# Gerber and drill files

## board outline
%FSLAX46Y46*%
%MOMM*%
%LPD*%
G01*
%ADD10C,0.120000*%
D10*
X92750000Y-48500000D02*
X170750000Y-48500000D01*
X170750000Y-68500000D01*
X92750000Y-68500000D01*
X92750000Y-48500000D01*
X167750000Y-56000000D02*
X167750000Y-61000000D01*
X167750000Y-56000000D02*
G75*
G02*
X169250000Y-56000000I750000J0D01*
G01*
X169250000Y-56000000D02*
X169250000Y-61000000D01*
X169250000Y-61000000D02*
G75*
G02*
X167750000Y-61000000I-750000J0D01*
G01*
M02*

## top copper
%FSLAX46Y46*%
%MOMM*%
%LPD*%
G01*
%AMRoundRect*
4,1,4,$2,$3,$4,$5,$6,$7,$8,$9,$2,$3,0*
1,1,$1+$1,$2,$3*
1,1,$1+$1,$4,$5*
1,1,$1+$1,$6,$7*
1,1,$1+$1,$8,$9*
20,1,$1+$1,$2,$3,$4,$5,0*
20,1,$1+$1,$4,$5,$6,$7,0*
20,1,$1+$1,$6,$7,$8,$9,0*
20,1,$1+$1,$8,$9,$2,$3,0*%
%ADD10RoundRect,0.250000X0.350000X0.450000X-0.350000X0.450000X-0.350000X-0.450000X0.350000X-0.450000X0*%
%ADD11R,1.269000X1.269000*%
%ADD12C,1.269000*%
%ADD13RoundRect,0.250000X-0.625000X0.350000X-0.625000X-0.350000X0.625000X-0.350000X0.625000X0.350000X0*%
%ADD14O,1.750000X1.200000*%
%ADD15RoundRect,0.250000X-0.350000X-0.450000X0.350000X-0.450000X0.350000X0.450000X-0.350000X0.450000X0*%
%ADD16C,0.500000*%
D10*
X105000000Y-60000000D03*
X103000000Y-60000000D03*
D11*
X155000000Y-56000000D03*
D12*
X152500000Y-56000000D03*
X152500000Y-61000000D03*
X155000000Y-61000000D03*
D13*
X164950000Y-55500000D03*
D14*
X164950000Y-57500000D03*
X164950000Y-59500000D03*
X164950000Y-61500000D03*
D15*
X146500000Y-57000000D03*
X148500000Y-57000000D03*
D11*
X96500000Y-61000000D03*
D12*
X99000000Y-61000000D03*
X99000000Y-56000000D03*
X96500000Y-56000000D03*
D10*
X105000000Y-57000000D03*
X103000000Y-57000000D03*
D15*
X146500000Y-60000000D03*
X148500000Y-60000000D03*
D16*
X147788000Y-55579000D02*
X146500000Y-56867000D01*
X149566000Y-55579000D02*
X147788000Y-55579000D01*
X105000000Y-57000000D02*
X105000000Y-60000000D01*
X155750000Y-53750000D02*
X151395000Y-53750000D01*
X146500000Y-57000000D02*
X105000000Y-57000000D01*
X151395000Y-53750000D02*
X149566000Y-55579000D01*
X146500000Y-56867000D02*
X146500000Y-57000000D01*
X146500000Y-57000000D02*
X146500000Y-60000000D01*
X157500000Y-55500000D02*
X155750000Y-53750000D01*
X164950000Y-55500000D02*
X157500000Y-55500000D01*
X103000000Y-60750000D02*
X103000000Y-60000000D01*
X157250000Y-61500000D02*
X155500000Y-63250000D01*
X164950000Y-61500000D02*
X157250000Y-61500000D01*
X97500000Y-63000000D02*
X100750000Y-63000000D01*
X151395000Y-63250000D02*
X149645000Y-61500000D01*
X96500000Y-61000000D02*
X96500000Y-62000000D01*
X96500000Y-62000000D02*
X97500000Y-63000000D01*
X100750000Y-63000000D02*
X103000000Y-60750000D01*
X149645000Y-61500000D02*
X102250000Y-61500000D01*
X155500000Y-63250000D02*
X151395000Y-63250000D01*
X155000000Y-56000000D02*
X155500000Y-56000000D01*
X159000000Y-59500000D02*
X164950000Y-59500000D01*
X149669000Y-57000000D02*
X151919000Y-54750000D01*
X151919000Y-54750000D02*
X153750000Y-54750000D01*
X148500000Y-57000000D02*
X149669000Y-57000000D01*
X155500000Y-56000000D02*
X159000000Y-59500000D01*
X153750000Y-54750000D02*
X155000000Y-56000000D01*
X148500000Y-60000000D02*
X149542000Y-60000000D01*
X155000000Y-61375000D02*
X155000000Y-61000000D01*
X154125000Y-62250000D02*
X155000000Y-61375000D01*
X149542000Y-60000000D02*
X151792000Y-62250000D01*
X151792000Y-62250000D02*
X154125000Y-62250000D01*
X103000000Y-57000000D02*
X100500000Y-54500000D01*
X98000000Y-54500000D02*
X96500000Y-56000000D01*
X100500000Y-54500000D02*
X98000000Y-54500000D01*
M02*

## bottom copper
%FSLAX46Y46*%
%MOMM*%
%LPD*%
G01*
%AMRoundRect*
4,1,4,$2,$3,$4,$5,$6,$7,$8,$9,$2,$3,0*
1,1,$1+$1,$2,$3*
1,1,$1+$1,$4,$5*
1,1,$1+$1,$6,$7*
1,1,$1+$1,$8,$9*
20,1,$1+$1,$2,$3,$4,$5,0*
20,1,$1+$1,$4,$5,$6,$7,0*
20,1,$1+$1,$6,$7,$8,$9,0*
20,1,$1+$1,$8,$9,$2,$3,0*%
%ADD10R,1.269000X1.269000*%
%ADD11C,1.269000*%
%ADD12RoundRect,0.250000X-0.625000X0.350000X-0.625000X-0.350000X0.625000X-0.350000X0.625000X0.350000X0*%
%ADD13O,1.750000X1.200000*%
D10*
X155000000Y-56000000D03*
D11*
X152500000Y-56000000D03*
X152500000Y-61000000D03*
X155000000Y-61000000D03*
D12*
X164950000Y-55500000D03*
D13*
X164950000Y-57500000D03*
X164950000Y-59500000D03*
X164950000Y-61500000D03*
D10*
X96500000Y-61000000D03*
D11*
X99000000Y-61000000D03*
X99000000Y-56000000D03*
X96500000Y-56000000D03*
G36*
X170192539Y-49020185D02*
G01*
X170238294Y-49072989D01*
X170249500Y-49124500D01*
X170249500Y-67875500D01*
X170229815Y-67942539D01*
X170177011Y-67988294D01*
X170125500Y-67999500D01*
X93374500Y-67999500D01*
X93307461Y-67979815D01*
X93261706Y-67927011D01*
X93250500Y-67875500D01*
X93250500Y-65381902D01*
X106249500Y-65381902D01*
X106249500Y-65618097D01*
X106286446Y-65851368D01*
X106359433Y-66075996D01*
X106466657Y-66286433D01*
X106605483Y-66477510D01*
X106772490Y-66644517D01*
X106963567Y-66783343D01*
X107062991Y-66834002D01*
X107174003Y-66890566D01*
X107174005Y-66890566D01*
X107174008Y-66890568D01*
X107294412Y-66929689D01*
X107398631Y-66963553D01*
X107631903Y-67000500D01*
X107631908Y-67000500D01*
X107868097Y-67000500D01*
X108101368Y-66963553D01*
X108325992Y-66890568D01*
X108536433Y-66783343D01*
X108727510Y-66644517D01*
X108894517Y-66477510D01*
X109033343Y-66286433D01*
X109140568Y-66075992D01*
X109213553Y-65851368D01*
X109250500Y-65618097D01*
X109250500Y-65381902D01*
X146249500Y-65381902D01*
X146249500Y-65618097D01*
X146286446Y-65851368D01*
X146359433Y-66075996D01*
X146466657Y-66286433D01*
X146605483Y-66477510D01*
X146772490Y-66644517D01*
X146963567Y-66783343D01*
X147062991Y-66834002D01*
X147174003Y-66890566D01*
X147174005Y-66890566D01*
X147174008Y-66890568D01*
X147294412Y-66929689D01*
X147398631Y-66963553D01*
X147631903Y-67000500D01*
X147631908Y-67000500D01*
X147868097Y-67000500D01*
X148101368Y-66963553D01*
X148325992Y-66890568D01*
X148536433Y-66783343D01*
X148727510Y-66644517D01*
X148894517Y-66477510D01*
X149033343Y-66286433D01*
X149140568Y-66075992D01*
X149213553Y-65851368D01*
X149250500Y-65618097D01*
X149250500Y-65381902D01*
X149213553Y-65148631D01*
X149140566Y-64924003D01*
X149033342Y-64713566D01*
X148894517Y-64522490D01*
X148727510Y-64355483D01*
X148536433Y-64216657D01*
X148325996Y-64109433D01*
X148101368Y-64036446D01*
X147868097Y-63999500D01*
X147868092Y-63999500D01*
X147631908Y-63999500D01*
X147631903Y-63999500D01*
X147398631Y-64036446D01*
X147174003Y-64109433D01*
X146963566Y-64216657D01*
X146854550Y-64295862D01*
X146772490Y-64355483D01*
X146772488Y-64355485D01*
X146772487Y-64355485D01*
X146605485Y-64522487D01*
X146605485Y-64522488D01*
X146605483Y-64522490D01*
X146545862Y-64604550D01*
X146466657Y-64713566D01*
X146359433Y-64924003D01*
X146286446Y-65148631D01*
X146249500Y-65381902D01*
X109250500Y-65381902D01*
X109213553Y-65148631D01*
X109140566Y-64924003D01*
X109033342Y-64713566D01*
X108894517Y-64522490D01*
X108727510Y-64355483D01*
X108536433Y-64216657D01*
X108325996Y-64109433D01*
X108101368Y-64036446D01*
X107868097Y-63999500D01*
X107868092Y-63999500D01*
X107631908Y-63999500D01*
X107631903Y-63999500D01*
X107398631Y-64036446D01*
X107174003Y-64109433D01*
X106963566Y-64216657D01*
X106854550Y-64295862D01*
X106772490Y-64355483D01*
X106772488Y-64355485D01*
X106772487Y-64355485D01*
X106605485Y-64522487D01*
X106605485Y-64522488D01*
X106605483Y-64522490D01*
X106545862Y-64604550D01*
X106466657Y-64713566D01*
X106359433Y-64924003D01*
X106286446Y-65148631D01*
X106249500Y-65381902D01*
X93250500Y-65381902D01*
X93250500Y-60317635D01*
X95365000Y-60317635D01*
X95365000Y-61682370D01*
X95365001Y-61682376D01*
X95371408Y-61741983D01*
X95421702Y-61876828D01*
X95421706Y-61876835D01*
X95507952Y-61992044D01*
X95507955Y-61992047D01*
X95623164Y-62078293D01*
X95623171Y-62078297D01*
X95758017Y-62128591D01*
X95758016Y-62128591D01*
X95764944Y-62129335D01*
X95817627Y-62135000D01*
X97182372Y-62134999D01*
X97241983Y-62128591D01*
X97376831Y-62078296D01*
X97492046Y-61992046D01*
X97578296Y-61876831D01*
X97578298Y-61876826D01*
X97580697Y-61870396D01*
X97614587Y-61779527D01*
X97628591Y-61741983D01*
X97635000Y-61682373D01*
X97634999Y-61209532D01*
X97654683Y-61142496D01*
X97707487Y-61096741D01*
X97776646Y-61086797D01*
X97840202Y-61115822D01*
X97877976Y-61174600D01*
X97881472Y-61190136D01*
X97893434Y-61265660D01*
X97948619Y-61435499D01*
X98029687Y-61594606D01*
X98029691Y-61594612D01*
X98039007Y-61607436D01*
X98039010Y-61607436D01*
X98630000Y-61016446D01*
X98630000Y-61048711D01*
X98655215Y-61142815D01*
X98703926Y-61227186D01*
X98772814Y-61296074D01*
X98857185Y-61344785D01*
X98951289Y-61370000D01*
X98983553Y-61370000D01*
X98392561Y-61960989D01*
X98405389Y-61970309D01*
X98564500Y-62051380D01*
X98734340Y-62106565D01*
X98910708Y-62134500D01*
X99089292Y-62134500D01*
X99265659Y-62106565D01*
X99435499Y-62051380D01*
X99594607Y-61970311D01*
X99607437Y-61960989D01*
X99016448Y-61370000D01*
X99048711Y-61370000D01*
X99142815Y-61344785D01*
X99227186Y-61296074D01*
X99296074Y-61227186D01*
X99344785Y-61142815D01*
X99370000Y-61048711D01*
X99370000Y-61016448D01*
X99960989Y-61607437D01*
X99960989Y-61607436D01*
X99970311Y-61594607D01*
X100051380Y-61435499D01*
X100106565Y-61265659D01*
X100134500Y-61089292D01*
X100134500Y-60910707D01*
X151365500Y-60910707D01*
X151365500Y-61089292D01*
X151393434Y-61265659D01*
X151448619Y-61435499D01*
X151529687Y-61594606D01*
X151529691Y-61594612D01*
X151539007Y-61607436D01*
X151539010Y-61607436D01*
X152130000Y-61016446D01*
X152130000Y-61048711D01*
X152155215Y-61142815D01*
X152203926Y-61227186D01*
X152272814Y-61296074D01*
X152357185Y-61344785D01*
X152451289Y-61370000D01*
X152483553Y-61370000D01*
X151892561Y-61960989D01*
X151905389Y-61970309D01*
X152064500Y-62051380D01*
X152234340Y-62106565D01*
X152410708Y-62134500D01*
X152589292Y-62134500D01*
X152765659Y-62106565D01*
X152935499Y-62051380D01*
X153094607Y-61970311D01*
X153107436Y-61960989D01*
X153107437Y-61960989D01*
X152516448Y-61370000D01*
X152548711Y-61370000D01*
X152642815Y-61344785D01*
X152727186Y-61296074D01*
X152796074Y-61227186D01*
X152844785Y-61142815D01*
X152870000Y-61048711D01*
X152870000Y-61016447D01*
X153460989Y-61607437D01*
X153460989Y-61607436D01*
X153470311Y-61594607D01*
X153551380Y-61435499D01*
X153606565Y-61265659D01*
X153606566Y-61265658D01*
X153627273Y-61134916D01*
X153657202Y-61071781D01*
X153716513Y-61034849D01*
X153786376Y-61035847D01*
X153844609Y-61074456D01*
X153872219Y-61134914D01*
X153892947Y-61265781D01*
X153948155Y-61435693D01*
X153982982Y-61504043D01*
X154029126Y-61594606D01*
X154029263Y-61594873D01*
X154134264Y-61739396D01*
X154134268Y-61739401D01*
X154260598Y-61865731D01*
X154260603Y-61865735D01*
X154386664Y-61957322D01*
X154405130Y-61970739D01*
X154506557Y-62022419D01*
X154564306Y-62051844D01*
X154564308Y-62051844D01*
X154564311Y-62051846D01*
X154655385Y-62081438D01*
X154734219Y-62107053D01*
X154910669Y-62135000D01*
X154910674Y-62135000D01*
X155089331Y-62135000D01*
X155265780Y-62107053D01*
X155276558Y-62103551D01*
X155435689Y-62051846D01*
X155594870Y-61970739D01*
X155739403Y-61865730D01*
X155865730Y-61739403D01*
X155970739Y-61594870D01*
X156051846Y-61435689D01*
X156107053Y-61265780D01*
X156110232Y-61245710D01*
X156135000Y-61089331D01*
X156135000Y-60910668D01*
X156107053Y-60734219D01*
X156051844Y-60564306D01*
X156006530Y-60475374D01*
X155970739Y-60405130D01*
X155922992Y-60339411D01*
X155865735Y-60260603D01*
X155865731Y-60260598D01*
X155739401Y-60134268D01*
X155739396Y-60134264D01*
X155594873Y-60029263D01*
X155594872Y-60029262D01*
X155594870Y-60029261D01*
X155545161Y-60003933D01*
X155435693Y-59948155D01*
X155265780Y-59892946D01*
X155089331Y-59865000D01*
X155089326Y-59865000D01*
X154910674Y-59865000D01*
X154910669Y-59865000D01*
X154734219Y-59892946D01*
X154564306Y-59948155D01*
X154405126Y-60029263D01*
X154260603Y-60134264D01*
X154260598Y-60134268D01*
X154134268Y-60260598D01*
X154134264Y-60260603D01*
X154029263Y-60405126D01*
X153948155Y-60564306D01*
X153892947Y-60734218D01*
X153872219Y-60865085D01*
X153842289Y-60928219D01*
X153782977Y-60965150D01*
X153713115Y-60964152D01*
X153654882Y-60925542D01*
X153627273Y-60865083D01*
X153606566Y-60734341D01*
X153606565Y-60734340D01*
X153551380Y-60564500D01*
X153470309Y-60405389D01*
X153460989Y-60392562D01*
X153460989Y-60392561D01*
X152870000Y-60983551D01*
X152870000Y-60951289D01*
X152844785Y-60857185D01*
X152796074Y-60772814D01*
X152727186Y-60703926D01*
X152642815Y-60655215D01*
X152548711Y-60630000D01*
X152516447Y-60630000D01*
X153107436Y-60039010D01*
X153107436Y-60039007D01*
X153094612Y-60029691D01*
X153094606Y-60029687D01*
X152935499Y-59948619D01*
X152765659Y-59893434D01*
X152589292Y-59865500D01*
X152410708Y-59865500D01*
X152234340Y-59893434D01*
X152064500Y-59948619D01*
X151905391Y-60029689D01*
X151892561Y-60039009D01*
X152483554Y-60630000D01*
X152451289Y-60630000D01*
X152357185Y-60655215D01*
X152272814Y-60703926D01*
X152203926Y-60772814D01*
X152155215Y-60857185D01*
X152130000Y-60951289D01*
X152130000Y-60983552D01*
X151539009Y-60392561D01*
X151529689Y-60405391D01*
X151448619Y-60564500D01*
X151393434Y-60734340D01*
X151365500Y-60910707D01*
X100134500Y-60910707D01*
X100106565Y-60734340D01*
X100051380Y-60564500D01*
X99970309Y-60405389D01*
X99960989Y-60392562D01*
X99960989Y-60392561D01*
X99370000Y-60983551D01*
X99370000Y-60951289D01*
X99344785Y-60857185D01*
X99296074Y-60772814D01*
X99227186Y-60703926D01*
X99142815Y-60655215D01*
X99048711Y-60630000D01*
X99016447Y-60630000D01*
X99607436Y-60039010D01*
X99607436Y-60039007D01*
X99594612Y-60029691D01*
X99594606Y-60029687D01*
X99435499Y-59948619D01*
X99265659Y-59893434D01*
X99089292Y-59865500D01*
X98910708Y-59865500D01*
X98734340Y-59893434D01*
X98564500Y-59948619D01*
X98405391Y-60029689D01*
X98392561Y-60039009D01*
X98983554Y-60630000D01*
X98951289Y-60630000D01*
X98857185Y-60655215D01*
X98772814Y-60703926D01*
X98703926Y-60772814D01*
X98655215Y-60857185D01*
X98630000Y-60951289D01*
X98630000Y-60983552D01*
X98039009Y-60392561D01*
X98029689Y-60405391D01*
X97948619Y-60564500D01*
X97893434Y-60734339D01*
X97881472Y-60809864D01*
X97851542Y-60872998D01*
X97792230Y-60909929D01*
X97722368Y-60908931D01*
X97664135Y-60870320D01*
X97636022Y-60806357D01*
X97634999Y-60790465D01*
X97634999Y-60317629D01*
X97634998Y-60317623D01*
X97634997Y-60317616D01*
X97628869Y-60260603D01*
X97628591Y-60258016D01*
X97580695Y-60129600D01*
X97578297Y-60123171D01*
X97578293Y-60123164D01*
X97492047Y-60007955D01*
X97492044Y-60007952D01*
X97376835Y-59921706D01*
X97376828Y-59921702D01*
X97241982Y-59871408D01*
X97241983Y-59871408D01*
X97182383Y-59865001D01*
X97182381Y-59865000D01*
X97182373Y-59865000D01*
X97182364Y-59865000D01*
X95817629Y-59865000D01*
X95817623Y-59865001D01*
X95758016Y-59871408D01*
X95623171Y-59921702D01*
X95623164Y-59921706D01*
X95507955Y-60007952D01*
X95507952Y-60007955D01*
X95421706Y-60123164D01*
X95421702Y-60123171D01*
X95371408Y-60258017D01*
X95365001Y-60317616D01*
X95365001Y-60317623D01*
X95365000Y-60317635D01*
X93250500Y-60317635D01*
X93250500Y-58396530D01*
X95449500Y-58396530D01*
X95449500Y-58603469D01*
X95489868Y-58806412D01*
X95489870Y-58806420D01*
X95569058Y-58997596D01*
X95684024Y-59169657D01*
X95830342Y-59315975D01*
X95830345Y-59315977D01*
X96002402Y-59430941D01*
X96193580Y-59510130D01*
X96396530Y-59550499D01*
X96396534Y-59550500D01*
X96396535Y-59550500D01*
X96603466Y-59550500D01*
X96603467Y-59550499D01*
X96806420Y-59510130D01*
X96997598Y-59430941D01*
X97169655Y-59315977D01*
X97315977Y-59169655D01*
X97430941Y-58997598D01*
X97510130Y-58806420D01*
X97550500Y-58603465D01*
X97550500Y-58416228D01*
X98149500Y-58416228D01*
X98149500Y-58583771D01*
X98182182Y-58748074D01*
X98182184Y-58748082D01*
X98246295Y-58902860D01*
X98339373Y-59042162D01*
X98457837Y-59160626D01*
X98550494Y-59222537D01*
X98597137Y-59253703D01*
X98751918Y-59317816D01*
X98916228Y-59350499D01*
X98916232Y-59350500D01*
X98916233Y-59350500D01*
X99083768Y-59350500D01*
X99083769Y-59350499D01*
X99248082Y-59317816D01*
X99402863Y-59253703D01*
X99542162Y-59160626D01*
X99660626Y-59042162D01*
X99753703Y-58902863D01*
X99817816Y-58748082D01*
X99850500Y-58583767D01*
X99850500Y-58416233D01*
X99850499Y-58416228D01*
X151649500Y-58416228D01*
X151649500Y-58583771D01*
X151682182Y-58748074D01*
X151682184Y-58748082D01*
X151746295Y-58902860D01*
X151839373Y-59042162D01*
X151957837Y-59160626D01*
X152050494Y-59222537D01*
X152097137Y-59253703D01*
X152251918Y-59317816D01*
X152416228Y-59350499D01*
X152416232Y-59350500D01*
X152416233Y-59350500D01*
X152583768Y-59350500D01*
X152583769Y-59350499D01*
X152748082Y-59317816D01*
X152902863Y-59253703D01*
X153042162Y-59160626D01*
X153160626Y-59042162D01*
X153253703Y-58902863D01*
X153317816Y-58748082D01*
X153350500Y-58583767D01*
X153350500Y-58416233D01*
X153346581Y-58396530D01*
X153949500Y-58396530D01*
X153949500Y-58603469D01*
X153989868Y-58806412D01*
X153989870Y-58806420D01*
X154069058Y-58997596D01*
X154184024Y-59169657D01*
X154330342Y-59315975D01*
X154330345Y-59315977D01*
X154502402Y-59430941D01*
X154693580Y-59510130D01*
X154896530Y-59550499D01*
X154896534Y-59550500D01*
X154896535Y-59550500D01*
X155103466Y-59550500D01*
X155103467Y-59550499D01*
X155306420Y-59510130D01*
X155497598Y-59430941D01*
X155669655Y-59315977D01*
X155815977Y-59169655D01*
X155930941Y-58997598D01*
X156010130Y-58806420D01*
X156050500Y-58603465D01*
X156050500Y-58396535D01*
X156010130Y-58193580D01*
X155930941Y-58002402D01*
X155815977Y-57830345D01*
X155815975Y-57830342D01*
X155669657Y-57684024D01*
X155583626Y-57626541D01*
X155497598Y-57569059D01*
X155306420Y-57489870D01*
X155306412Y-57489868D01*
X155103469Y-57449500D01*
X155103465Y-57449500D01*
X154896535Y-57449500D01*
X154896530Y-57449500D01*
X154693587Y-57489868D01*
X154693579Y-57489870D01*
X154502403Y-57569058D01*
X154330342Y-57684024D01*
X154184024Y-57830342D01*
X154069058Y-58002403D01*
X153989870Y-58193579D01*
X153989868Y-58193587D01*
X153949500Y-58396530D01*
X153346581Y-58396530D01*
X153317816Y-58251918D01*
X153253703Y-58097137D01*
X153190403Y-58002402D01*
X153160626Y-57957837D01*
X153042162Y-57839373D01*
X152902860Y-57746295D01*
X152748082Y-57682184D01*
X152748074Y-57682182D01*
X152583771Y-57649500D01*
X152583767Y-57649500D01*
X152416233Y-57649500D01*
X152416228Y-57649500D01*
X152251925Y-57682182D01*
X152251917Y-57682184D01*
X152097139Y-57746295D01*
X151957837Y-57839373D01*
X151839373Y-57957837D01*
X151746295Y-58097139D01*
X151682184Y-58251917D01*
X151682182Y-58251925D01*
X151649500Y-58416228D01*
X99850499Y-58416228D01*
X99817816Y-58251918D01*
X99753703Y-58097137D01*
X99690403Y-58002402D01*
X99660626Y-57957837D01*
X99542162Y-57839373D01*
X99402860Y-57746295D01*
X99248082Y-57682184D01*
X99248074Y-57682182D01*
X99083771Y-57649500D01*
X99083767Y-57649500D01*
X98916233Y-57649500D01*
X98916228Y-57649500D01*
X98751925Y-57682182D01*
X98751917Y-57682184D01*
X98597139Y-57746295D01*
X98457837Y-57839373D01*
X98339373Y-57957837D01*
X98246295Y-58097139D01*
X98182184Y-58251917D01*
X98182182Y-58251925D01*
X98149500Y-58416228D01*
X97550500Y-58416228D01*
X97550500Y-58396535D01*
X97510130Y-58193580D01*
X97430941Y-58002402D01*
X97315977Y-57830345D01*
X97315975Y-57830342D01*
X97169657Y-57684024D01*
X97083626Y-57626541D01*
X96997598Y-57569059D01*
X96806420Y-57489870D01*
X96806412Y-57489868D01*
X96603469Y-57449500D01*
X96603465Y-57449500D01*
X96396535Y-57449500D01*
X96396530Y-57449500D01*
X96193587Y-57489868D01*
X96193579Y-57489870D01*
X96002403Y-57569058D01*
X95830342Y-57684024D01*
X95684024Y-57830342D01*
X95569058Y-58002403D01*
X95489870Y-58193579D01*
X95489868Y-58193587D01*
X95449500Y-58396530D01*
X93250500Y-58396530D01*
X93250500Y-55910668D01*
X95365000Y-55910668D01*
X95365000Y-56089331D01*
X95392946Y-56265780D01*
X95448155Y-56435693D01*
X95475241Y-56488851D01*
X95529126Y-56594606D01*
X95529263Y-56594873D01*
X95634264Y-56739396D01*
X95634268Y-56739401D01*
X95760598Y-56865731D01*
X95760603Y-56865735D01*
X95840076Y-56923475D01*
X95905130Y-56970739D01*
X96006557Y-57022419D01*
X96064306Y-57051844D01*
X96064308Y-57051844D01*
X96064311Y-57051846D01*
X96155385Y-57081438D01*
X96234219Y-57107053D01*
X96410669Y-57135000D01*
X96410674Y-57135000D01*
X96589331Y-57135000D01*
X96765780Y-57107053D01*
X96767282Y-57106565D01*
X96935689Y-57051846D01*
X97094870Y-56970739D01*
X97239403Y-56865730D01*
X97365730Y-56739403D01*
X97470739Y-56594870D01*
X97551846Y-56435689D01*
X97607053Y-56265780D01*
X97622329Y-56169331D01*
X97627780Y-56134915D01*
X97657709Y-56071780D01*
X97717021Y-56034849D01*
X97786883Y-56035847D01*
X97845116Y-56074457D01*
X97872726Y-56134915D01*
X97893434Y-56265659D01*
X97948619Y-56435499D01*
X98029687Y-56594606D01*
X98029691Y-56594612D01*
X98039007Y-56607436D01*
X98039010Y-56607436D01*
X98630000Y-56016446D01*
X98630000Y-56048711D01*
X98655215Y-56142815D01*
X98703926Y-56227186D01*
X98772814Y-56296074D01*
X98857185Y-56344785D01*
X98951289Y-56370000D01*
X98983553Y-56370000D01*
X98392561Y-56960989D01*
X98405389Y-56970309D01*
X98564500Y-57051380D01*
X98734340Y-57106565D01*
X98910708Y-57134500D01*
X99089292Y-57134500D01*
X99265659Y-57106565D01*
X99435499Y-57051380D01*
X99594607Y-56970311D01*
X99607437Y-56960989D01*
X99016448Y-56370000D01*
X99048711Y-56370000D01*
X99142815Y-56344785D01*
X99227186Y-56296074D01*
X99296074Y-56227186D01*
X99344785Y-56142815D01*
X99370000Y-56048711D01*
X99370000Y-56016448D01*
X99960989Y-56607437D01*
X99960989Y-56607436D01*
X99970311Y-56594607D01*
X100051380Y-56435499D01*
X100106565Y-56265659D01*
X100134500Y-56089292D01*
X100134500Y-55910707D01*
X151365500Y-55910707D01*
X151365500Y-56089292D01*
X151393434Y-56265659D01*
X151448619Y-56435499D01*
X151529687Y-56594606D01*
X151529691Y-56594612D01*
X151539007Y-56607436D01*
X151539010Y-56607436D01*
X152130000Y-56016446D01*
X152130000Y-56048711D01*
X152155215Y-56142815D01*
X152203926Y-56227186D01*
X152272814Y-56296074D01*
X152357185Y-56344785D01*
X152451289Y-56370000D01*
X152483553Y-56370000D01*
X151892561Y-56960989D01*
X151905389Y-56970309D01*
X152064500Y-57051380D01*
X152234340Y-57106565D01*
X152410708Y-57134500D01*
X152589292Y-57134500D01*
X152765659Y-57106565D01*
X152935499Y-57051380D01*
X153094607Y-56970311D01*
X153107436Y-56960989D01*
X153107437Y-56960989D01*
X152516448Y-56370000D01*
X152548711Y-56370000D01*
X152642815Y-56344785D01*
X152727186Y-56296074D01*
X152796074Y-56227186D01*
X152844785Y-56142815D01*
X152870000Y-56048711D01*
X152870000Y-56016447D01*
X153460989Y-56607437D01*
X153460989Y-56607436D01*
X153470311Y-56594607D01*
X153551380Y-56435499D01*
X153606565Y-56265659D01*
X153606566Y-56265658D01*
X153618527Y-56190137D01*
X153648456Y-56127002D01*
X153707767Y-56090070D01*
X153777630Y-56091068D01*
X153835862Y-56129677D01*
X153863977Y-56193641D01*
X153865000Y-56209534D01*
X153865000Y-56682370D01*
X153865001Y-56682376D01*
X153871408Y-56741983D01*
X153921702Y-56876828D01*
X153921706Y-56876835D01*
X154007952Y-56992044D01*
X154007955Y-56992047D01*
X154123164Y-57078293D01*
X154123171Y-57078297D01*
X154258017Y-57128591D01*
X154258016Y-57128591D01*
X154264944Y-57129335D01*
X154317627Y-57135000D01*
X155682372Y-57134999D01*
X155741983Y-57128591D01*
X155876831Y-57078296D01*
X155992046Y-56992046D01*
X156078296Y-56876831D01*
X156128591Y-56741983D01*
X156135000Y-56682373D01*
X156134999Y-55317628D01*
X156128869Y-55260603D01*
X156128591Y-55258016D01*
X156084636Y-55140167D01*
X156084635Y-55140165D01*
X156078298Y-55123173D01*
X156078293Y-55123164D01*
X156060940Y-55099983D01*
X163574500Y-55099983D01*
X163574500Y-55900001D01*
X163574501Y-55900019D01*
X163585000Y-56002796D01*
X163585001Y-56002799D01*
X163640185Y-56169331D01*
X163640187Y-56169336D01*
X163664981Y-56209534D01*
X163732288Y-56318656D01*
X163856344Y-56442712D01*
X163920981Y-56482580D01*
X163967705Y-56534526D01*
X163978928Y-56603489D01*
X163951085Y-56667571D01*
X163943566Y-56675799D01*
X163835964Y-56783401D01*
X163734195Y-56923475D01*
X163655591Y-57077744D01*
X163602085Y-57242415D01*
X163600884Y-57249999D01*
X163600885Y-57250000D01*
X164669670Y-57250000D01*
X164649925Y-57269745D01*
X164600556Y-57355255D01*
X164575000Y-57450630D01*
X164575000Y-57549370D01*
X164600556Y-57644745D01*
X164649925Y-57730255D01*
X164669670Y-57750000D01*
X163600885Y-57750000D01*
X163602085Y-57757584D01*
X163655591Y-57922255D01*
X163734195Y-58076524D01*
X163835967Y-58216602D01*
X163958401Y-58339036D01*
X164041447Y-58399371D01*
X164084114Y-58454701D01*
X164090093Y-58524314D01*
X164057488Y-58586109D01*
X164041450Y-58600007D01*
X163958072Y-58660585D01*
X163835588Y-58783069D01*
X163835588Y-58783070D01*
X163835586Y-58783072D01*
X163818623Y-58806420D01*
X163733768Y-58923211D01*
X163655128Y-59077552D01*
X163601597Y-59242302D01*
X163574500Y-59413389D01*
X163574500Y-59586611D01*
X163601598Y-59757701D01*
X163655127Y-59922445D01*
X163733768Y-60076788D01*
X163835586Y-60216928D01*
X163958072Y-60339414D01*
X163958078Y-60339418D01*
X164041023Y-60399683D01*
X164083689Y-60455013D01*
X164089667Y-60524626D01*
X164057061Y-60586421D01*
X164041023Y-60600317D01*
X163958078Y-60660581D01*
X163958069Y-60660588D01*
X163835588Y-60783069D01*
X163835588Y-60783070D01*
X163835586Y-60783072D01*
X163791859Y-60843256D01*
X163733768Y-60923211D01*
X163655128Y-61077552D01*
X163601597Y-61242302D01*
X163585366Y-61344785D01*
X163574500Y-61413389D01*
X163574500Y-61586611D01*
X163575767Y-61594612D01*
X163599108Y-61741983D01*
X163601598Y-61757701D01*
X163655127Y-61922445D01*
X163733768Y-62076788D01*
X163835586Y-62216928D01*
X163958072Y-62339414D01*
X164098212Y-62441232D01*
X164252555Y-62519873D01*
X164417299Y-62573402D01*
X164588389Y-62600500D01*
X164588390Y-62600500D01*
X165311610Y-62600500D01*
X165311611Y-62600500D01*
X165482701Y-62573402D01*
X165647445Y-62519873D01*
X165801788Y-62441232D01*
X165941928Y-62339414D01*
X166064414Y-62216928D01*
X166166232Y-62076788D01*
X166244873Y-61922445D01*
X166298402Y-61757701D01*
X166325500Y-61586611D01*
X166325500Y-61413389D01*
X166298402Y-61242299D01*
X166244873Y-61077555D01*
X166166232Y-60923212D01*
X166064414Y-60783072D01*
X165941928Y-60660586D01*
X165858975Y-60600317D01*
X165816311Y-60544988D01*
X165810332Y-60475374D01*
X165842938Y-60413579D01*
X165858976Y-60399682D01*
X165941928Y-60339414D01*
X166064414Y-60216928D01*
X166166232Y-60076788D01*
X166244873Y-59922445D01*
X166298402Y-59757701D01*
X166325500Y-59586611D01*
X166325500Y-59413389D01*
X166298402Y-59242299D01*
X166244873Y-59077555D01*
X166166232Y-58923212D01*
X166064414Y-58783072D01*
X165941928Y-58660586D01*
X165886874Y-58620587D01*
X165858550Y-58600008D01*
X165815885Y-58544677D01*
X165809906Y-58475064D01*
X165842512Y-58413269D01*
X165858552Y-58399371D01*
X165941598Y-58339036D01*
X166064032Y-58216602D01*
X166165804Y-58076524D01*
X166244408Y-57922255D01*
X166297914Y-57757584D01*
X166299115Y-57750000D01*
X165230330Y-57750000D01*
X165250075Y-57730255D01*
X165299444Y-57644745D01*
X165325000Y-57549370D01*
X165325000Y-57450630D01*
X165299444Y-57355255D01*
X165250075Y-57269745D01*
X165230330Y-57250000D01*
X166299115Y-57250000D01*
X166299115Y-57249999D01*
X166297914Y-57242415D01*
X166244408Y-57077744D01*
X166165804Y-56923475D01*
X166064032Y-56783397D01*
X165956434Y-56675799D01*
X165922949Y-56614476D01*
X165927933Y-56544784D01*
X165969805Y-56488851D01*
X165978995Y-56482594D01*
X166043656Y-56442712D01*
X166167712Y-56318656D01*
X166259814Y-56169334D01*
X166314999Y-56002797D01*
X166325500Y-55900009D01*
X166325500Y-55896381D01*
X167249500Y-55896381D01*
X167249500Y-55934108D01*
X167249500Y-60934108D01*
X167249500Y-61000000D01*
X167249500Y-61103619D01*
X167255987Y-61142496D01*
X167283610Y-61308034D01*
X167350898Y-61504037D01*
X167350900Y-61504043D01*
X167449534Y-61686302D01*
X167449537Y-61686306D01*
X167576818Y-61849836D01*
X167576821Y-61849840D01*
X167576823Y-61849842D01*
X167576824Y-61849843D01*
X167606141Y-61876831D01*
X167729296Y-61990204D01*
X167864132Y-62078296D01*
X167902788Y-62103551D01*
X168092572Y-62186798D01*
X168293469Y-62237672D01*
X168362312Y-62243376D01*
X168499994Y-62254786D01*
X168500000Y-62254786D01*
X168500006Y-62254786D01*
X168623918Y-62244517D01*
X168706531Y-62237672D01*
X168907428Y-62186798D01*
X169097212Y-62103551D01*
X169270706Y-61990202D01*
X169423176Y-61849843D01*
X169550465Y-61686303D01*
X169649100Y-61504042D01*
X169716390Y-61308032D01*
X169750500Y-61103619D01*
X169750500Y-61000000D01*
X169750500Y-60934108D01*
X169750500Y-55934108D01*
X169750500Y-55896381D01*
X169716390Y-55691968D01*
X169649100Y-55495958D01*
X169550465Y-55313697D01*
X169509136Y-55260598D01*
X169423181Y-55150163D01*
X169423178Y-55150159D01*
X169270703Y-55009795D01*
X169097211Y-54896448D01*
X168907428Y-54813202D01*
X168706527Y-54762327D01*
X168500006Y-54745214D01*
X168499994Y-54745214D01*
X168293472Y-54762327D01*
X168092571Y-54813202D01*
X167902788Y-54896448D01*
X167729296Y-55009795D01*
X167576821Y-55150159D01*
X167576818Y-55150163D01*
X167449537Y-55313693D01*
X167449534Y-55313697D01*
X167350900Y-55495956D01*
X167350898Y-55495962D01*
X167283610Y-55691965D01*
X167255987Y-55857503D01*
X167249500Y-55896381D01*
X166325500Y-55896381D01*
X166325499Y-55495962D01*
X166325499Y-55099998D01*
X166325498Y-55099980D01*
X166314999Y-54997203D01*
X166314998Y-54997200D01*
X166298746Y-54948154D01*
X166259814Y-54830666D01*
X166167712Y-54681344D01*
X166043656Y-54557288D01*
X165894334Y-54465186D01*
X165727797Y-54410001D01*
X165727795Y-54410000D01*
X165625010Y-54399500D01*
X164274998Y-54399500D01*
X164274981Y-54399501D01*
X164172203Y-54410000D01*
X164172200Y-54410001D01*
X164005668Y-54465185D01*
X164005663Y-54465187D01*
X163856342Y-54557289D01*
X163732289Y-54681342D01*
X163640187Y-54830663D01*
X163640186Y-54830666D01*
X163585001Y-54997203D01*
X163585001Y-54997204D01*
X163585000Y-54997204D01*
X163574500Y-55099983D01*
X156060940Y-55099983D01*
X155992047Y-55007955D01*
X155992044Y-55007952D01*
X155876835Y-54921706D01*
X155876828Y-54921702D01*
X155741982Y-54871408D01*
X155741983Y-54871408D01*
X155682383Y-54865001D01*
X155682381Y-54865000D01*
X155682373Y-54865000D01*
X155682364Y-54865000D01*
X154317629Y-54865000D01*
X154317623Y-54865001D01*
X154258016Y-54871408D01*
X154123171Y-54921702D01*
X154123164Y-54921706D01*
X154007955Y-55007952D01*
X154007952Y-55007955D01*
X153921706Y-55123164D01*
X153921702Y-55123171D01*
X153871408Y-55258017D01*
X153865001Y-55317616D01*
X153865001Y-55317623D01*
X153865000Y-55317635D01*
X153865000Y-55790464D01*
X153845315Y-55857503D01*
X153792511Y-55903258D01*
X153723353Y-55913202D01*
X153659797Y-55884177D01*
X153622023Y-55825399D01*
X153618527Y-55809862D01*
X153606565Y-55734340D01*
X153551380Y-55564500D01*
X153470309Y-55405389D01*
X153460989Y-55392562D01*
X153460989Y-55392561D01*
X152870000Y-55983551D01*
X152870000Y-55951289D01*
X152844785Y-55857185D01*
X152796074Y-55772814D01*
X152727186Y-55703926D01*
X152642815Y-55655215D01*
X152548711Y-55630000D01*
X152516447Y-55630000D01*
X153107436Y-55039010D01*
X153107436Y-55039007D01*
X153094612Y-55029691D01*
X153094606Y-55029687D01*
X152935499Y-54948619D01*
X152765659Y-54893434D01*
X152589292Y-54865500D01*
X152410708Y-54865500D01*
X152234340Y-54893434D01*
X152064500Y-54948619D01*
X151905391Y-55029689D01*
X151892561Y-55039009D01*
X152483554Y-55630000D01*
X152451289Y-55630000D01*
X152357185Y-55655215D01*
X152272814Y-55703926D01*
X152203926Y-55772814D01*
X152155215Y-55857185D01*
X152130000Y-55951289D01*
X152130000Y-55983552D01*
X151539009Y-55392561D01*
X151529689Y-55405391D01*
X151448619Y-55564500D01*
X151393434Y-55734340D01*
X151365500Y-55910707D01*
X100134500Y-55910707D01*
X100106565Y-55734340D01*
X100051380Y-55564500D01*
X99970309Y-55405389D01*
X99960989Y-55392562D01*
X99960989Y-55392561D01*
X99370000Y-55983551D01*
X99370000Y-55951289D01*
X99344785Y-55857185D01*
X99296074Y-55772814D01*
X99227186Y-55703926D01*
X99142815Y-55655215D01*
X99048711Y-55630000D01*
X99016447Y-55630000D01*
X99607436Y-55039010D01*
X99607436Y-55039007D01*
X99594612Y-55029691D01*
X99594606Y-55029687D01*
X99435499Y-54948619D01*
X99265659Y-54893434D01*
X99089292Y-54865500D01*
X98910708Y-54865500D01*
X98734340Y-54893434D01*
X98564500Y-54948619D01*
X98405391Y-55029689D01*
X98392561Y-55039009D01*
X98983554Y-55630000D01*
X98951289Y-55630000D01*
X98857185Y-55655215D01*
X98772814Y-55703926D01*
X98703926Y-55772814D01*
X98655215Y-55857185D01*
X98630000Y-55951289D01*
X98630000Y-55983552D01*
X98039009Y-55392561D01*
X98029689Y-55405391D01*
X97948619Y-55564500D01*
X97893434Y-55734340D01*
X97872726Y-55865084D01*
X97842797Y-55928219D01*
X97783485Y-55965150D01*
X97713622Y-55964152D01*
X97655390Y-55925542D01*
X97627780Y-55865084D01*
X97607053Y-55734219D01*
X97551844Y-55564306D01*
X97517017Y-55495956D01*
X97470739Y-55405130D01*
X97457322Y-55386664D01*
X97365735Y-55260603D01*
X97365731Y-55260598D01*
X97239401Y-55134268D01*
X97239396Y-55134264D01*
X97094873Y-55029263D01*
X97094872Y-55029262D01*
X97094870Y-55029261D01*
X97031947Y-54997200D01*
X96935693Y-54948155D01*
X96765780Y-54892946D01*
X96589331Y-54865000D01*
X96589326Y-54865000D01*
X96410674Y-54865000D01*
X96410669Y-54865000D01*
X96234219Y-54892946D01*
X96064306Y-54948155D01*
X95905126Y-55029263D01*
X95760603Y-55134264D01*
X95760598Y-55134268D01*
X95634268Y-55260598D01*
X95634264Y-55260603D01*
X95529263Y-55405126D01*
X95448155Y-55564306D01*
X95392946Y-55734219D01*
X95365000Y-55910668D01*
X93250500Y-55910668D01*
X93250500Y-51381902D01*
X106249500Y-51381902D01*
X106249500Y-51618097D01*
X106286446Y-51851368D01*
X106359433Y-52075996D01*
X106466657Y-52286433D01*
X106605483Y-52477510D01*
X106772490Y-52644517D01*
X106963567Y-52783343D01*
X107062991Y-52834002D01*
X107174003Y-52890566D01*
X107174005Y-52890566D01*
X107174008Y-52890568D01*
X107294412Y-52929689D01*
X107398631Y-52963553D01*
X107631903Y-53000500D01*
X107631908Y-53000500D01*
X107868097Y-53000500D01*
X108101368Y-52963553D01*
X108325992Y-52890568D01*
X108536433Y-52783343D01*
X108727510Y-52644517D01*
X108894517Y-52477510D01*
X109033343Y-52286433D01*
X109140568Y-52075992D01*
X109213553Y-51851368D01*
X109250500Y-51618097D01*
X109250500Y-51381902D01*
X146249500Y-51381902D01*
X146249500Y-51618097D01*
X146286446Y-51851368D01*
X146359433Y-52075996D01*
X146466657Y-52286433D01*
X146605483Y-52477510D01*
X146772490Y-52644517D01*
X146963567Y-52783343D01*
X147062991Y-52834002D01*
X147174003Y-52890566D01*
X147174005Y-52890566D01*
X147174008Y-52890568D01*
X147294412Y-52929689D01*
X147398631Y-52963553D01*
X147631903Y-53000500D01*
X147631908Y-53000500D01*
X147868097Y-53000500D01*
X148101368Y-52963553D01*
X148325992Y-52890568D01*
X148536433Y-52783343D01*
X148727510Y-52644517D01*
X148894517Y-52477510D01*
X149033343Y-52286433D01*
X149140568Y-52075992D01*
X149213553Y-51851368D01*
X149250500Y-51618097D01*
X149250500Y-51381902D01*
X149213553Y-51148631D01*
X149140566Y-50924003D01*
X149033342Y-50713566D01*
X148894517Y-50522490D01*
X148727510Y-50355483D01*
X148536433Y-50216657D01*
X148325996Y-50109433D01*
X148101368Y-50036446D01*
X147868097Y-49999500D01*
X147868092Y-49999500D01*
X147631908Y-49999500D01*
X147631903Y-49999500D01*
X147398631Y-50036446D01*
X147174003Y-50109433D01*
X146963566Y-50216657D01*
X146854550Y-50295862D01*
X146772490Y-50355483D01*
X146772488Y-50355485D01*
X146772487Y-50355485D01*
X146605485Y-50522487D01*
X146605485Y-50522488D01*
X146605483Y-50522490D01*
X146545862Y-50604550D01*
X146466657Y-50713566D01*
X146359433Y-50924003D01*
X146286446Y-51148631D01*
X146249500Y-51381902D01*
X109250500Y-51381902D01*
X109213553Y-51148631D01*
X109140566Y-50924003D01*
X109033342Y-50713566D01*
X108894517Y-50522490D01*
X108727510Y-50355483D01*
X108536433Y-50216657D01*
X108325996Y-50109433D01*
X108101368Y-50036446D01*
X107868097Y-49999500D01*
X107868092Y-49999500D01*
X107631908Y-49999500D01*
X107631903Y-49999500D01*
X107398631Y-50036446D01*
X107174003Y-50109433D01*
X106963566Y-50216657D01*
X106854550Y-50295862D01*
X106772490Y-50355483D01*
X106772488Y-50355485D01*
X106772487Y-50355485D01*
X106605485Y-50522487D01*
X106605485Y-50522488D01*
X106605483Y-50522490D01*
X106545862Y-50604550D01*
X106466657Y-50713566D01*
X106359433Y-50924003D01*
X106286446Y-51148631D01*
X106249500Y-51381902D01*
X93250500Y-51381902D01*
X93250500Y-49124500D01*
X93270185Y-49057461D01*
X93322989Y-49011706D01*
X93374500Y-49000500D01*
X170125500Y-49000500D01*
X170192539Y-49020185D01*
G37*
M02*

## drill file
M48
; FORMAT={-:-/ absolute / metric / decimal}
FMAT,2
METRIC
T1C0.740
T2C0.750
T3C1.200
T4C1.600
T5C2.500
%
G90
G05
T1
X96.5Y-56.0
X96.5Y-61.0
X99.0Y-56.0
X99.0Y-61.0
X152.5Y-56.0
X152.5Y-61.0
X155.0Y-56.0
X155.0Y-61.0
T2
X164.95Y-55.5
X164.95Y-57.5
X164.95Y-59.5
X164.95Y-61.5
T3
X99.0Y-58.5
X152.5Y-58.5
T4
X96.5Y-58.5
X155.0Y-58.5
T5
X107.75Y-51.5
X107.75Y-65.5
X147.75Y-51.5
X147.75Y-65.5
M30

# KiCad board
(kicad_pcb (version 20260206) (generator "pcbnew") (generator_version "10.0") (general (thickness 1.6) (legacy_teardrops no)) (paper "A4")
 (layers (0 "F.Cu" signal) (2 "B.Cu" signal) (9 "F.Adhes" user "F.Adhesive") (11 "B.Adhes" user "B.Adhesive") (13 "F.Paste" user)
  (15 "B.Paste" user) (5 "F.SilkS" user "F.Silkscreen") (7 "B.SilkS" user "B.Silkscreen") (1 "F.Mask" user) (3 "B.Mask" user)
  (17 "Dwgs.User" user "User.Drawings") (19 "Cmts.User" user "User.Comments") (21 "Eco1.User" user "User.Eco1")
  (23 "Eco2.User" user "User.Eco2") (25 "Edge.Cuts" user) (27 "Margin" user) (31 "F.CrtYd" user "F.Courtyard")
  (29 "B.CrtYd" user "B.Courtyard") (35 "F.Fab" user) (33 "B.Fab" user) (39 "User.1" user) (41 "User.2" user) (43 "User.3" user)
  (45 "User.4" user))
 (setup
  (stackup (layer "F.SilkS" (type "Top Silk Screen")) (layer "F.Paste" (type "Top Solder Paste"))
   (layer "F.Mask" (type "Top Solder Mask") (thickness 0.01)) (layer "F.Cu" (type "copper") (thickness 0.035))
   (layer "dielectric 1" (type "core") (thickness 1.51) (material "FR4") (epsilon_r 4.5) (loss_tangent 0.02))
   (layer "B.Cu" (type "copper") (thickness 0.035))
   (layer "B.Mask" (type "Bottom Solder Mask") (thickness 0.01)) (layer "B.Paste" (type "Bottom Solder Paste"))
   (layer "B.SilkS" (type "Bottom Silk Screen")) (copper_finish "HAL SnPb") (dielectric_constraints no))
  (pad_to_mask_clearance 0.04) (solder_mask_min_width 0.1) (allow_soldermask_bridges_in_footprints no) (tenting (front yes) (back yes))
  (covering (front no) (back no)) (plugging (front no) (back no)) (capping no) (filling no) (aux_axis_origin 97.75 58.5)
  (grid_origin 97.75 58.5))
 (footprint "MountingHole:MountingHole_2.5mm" (layer "F.Cu") (at 107.75 51.5)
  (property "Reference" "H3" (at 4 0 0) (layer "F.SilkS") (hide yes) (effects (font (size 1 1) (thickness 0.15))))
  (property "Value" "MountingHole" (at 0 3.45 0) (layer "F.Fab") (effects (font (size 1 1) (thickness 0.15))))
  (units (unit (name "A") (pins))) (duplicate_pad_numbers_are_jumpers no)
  (pad "" np_thru_hole circle (at 0 0) (size 2.5 2.5) (drill 2.5) (layers "*.Cu" "*.Mask")))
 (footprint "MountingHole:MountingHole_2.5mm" (layer "F.Cu") (at 107.75 65.5)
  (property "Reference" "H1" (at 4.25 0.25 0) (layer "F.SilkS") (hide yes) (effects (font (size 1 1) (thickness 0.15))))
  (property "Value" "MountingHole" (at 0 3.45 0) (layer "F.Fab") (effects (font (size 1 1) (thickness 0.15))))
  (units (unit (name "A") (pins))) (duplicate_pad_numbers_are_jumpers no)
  (pad "" np_thru_hole circle (at 0 0) (size 2.5 2.5) (drill 2.5) (layers "*.Cu" "*.Mask")))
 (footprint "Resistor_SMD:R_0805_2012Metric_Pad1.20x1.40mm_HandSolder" (layer "F.Cu") (at 104 60 180)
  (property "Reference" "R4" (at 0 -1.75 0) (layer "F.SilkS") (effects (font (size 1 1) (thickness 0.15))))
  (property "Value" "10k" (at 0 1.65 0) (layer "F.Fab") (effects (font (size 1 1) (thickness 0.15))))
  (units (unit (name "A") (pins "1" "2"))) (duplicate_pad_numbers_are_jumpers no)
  (pad "1" smd roundrect (at -1 0 180) (size 1.2 1.4) (layers "F.Cu" "F.Mask" "F.Paste") (roundrect_rratio 0.208333) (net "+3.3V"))
  (pad "2" smd roundrect (at 1 0 180) (size 1.2 1.4) (layers "F.Cu" "F.Mask" "F.Paste") (roundrect_rratio 0.208333) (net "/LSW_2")))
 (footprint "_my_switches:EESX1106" (layer "F.Cu") (at 155 56 -90)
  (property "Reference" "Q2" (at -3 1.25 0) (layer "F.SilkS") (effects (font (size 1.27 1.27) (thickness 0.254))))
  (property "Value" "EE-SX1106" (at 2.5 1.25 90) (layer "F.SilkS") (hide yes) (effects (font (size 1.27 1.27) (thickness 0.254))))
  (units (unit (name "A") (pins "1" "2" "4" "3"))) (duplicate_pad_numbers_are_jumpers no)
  (pad "" np_thru_hole circle (at 2.5 0 270) (size 1.6 1.6) (drill 1.6) (layers "*.Cu" "*.Mask"))
  (pad "" np_thru_hole circle (at 2.5 2.5 270) (size 1.2 1.2) (drill 1.2) (layers "*.Cu" "*.Mask"))
  (pad "1" thru_hole rect (at 0 0 270) (size 1.269 1.269) (drill 0.74) (layers "*.Cu" "*.Mask") (remove_unused_layers no) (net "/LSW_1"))
  (pad "2" thru_hole circle (at 0 2.5 270) (size 1.269 1.269) (drill 0.74) (layers "*.Cu" "*.Mask") (remove_unused_layers no) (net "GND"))
  (pad "3" thru_hole circle (at 5 2.5 270) (size 1.269 1.269) (drill 0.74) (layers "*.Cu" "*.Mask") (remove_unused_layers no) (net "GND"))
  (pad "4" thru_hole circle (at 5 0 270) (size 1.269 1.269) (drill 0.74) (layers "*.Cu" "*.Mask") (remove_unused_layers no)
   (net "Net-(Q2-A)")))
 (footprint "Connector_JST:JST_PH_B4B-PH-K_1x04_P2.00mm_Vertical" (layer "F.Cu") (at 164.95 55.5 -90)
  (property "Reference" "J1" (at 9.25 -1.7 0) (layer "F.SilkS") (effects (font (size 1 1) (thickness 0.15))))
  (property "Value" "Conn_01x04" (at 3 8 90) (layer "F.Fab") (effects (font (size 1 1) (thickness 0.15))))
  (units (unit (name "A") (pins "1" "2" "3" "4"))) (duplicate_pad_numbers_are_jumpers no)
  (pad "1" thru_hole roundrect (at 0 0 270) (size 1.2 1.75) (drill 0.75) (layers "*.Cu" "*.Mask") (remove_unused_layers no)
   (roundrect_rratio 0.208333) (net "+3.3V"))
  (pad "2" thru_hole oval (at 2 0 270) (size 1.2 1.75) (drill 0.75) (layers "*.Cu" "*.Mask") (remove_unused_layers no) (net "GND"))
  (pad "3" thru_hole oval (at 4 0 270) (size 1.2 1.75) (drill 0.75) (layers "*.Cu" "*.Mask") (remove_unused_layers no) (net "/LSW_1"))
  (pad "4" thru_hole oval (at 6 0 270) (size 1.2 1.75) (drill 0.75) (layers "*.Cu" "*.Mask") (remove_unused_layers no) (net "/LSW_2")))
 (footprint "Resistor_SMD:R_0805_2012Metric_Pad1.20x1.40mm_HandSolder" (layer "F.Cu") (at 147.5 57)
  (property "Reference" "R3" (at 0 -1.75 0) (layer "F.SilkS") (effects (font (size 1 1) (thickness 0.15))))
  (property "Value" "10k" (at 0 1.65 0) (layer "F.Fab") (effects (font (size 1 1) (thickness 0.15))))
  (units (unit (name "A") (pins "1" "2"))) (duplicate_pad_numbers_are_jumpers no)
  (pad "1" smd roundrect (at -1 0) (size 1.2 1.4) (layers "F.Cu" "F.Mask" "F.Paste") (roundrect_rratio 0.208333) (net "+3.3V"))
  (pad "2" smd roundrect (at 1 0) (size 1.2 1.4) (layers "F.Cu" "F.Mask" "F.Paste") (roundrect_rratio 0.208333) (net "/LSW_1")))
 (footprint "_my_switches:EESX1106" (layer "F.Cu") (at 96.5 61 90)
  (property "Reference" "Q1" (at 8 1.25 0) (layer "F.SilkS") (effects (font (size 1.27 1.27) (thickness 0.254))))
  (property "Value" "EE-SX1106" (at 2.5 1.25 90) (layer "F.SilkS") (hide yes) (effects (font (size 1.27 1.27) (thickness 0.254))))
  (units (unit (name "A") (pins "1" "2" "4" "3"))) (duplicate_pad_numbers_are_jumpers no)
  (pad "" np_thru_hole circle (at 2.5 0 90) (size 1.6 1.6) (drill 1.6) (layers "*.Cu" "*.Mask"))
  (pad "" np_thru_hole circle (at 2.5 2.5 90) (size 1.2 1.2) (drill 1.2) (layers "*.Cu" "*.Mask"))
  (pad "1" thru_hole rect (at 0 0 90) (size 1.269 1.269) (drill 0.74) (layers "*.Cu" "*.Mask") (remove_unused_layers no) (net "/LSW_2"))
  (pad "2" thru_hole circle (at 0 2.5 90) (size 1.269 1.269) (drill 0.74) (layers "*.Cu" "*.Mask") (remove_unused_layers no) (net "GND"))
  (pad "3" thru_hole circle (at 5 2.5 90) (size 1.269 1.269) (drill 0.74) (layers "*.Cu" "*.Mask") (remove_unused_layers no) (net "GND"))
  (pad "4" thru_hole circle (at 5 0 90) (size 1.269 1.269) (drill 0.74) (layers "*.Cu" "*.Mask") (remove_unused_layers no)
   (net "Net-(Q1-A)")))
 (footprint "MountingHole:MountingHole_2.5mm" (layer "F.Cu") (at 147.75 51.5)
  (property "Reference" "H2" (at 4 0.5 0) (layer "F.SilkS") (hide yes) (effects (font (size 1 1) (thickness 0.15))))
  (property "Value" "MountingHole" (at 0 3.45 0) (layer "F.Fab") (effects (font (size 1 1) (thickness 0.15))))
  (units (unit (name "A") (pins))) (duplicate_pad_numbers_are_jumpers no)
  (pad "" np_thru_hole circle (at 0 0) (size 2.5 2.5) (drill 2.5) (layers "*.Cu" "*.Mask")))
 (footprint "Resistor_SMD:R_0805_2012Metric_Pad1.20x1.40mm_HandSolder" (layer "F.Cu") (at 104 57 180)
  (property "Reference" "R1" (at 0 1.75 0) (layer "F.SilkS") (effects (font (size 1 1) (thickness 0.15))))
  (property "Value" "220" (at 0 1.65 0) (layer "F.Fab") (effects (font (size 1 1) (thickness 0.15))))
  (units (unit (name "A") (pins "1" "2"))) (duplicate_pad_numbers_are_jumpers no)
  (pad "1" smd roundrect (at -1 0 180) (size 1.2 1.4) (layers "F.Cu" "F.Mask" "F.Paste") (roundrect_rratio 0.208333) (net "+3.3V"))
  (pad "2" smd roundrect (at 1 0 180) (size 1.2 1.4) (layers "F.Cu" "F.Mask" "F.Paste") (roundrect_rratio 0.208333) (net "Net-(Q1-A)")))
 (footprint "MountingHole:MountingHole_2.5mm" (layer "F.Cu") (at 147.75 65.5)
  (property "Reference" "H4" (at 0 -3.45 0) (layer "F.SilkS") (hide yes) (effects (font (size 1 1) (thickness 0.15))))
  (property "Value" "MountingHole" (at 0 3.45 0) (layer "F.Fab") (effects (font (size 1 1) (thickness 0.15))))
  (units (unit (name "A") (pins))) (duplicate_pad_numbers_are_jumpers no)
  (pad "" np_thru_hole circle (at 0 0) (size 2.5 2.5) (drill 2.5) (layers "*.Cu" "*.Mask")))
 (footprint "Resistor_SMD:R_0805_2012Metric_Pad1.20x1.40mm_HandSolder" (layer "F.Cu") (at 147.5 60)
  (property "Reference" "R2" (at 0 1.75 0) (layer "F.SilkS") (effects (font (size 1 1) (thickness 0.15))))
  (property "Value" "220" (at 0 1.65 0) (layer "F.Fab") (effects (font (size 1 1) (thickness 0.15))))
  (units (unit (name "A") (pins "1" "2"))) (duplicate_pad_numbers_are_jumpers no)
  (pad "1" smd roundrect (at -1 0) (size 1.2 1.4) (layers "F.Cu" "F.Mask" "F.Paste") (roundrect_rratio 0.208333) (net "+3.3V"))
  (pad "2" smd roundrect (at 1 0) (size 1.2 1.4) (layers "F.Cu" "F.Mask" "F.Paste") (roundrect_rratio 0.208333) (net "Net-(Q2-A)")))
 (gr_rect (start 92.75 48.5) (end 170.75 68.5) (stroke (width 0.12) (type default)) (fill no) (layer "Edge.Cuts"))
 (gr_line (start 167.75 56) (end 167.75 61) (stroke (width 0.12) (type default)) (layer "Edge.Cuts"))
 (gr_arc (start 167.75 56) (mid 168.5 55.25) (end 169.25 56) (stroke (width 0.12) (type default)) (layer "Edge.Cuts"))
 (gr_line (start 169.25 56) (end 169.25 61) (stroke (width 0.12) (type default)) (layer "Edge.Cuts"))
 (gr_arc (start 169.25 61) (mid 168.5 61.75) (end 167.75 61) (stroke (width 0.12) (type default)) (layer "Edge.Cuts"))
 (segment (start 147.788 55.579) (end 146.5 56.867) (width 0.5) (layer "F.Cu") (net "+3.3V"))
 (segment (start 149.566 55.579) (end 147.788 55.579) (width 0.5) (layer "F.Cu") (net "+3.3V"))
 (segment (start 105 57) (end 105 60) (width 0.5) (layer "F.Cu") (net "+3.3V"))
 (segment (start 155.75 53.75) (end 151.395 53.75) (width 0.5) (layer "F.Cu") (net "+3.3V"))
 (segment (start 146.5 57) (end 105 57) (width 0.5) (layer "F.Cu") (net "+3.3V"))
 (segment (start 151.395 53.75) (end 149.566 55.579) (width 0.5) (layer "F.Cu") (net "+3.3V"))
 (segment (start 146.5 56.867) (end 146.5 57) (width 0.5) (layer "F.Cu") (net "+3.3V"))
 (segment (start 146.5 57) (end 146.5 60) (width 0.5) (layer "F.Cu") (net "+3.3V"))
 (segment (start 157.5 55.5) (end 155.75 53.75) (width 0.5) (layer "F.Cu") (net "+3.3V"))
 (segment (start 164.95 55.5) (end 157.5 55.5) (width 0.5) (layer "F.Cu") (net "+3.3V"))
 (segment (start 103 60.75) (end 103 60) (width 0.5) (layer "F.Cu") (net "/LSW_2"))
 (segment (start 157.25 61.5) (end 155.5 63.25) (width 0.5) (layer "F.Cu") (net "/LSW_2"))
 (segment (start 164.95 61.5) (end 157.25 61.5) (width 0.5) (layer "F.Cu") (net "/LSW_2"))
 (segment (start 97.5 63) (end 100.75 63) (width 0.5) (layer "F.Cu") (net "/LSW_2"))
 (segment (start 151.395 63.25) (end 149.645 61.5) (width 0.5) (layer "F.Cu") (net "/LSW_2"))
 (segment (start 96.5 61) (end 96.5 62) (width 0.5) (layer "F.Cu") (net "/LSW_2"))
 (segment (start 96.5 62) (end 97.5 63) (width 0.5) (layer "F.Cu") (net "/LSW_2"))
 (segment (start 100.75 63) (end 103 60.75) (width 0.5) (layer "F.Cu") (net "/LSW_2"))
 (segment (start 149.645 61.5) (end 102.25 61.5) (width 0.5) (layer "F.Cu") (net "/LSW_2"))
 (segment (start 155.5 63.25) (end 151.395 63.25) (width 0.5) (layer "F.Cu") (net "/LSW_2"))
 (segment (start 155 56) (end 155.5 56) (width 0.5) (layer "F.Cu") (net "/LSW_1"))
 (segment (start 159 59.5) (end 164.95 59.5) (width 0.5) (layer "F.Cu") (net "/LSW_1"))
 (segment (start 149.669 57) (end 151.919 54.75) (width 0.5) (layer "F.Cu") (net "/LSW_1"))
 (segment (start 151.919 54.75) (end 153.75 54.75) (width 0.5) (layer "F.Cu") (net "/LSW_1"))
 (segment (start 148.5 57) (end 149.669 57) (width 0.5) (layer "F.Cu") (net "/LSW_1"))
 (segment (start 155.5 56) (end 159 59.5) (width 0.5) (layer "F.Cu") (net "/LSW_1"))
 (segment (start 153.75 54.75) (end 155 56) (width 0.5) (layer "F.Cu") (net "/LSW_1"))
 (segment (start 148.5 60) (end 149.542 60) (width 0.5) (layer "F.Cu") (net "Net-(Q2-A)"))
 (segment (start 155 61.375) (end 155 61) (width 0.5) (layer "F.Cu") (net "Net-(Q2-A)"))
 (segment (start 154.125 62.25) (end 155 61.375) (width 0.5) (layer "F.Cu") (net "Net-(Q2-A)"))
 (segment (start 149.542 60) (end 151.792 62.25) (width 0.5) (layer "F.Cu") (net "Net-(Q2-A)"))
 (segment (start 151.792 62.25) (end 154.125 62.25) (width 0.5) (layer "F.Cu") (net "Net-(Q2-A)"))
 (segment (start 103 57) (end 100.5 54.5) (width 0.5) (layer "F.Cu") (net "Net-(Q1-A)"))
 (segment (start 98 54.5) (end 96.5 56) (width 0.5) (layer "F.Cu") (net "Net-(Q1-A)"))
 (segment (start 100.5 54.5) (end 98 54.5) (width 0.5) (layer "F.Cu") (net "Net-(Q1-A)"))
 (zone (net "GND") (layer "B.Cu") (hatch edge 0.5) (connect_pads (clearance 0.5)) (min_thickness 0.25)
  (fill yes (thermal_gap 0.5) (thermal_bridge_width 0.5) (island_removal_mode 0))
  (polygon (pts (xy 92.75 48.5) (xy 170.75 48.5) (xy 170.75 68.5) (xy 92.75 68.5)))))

